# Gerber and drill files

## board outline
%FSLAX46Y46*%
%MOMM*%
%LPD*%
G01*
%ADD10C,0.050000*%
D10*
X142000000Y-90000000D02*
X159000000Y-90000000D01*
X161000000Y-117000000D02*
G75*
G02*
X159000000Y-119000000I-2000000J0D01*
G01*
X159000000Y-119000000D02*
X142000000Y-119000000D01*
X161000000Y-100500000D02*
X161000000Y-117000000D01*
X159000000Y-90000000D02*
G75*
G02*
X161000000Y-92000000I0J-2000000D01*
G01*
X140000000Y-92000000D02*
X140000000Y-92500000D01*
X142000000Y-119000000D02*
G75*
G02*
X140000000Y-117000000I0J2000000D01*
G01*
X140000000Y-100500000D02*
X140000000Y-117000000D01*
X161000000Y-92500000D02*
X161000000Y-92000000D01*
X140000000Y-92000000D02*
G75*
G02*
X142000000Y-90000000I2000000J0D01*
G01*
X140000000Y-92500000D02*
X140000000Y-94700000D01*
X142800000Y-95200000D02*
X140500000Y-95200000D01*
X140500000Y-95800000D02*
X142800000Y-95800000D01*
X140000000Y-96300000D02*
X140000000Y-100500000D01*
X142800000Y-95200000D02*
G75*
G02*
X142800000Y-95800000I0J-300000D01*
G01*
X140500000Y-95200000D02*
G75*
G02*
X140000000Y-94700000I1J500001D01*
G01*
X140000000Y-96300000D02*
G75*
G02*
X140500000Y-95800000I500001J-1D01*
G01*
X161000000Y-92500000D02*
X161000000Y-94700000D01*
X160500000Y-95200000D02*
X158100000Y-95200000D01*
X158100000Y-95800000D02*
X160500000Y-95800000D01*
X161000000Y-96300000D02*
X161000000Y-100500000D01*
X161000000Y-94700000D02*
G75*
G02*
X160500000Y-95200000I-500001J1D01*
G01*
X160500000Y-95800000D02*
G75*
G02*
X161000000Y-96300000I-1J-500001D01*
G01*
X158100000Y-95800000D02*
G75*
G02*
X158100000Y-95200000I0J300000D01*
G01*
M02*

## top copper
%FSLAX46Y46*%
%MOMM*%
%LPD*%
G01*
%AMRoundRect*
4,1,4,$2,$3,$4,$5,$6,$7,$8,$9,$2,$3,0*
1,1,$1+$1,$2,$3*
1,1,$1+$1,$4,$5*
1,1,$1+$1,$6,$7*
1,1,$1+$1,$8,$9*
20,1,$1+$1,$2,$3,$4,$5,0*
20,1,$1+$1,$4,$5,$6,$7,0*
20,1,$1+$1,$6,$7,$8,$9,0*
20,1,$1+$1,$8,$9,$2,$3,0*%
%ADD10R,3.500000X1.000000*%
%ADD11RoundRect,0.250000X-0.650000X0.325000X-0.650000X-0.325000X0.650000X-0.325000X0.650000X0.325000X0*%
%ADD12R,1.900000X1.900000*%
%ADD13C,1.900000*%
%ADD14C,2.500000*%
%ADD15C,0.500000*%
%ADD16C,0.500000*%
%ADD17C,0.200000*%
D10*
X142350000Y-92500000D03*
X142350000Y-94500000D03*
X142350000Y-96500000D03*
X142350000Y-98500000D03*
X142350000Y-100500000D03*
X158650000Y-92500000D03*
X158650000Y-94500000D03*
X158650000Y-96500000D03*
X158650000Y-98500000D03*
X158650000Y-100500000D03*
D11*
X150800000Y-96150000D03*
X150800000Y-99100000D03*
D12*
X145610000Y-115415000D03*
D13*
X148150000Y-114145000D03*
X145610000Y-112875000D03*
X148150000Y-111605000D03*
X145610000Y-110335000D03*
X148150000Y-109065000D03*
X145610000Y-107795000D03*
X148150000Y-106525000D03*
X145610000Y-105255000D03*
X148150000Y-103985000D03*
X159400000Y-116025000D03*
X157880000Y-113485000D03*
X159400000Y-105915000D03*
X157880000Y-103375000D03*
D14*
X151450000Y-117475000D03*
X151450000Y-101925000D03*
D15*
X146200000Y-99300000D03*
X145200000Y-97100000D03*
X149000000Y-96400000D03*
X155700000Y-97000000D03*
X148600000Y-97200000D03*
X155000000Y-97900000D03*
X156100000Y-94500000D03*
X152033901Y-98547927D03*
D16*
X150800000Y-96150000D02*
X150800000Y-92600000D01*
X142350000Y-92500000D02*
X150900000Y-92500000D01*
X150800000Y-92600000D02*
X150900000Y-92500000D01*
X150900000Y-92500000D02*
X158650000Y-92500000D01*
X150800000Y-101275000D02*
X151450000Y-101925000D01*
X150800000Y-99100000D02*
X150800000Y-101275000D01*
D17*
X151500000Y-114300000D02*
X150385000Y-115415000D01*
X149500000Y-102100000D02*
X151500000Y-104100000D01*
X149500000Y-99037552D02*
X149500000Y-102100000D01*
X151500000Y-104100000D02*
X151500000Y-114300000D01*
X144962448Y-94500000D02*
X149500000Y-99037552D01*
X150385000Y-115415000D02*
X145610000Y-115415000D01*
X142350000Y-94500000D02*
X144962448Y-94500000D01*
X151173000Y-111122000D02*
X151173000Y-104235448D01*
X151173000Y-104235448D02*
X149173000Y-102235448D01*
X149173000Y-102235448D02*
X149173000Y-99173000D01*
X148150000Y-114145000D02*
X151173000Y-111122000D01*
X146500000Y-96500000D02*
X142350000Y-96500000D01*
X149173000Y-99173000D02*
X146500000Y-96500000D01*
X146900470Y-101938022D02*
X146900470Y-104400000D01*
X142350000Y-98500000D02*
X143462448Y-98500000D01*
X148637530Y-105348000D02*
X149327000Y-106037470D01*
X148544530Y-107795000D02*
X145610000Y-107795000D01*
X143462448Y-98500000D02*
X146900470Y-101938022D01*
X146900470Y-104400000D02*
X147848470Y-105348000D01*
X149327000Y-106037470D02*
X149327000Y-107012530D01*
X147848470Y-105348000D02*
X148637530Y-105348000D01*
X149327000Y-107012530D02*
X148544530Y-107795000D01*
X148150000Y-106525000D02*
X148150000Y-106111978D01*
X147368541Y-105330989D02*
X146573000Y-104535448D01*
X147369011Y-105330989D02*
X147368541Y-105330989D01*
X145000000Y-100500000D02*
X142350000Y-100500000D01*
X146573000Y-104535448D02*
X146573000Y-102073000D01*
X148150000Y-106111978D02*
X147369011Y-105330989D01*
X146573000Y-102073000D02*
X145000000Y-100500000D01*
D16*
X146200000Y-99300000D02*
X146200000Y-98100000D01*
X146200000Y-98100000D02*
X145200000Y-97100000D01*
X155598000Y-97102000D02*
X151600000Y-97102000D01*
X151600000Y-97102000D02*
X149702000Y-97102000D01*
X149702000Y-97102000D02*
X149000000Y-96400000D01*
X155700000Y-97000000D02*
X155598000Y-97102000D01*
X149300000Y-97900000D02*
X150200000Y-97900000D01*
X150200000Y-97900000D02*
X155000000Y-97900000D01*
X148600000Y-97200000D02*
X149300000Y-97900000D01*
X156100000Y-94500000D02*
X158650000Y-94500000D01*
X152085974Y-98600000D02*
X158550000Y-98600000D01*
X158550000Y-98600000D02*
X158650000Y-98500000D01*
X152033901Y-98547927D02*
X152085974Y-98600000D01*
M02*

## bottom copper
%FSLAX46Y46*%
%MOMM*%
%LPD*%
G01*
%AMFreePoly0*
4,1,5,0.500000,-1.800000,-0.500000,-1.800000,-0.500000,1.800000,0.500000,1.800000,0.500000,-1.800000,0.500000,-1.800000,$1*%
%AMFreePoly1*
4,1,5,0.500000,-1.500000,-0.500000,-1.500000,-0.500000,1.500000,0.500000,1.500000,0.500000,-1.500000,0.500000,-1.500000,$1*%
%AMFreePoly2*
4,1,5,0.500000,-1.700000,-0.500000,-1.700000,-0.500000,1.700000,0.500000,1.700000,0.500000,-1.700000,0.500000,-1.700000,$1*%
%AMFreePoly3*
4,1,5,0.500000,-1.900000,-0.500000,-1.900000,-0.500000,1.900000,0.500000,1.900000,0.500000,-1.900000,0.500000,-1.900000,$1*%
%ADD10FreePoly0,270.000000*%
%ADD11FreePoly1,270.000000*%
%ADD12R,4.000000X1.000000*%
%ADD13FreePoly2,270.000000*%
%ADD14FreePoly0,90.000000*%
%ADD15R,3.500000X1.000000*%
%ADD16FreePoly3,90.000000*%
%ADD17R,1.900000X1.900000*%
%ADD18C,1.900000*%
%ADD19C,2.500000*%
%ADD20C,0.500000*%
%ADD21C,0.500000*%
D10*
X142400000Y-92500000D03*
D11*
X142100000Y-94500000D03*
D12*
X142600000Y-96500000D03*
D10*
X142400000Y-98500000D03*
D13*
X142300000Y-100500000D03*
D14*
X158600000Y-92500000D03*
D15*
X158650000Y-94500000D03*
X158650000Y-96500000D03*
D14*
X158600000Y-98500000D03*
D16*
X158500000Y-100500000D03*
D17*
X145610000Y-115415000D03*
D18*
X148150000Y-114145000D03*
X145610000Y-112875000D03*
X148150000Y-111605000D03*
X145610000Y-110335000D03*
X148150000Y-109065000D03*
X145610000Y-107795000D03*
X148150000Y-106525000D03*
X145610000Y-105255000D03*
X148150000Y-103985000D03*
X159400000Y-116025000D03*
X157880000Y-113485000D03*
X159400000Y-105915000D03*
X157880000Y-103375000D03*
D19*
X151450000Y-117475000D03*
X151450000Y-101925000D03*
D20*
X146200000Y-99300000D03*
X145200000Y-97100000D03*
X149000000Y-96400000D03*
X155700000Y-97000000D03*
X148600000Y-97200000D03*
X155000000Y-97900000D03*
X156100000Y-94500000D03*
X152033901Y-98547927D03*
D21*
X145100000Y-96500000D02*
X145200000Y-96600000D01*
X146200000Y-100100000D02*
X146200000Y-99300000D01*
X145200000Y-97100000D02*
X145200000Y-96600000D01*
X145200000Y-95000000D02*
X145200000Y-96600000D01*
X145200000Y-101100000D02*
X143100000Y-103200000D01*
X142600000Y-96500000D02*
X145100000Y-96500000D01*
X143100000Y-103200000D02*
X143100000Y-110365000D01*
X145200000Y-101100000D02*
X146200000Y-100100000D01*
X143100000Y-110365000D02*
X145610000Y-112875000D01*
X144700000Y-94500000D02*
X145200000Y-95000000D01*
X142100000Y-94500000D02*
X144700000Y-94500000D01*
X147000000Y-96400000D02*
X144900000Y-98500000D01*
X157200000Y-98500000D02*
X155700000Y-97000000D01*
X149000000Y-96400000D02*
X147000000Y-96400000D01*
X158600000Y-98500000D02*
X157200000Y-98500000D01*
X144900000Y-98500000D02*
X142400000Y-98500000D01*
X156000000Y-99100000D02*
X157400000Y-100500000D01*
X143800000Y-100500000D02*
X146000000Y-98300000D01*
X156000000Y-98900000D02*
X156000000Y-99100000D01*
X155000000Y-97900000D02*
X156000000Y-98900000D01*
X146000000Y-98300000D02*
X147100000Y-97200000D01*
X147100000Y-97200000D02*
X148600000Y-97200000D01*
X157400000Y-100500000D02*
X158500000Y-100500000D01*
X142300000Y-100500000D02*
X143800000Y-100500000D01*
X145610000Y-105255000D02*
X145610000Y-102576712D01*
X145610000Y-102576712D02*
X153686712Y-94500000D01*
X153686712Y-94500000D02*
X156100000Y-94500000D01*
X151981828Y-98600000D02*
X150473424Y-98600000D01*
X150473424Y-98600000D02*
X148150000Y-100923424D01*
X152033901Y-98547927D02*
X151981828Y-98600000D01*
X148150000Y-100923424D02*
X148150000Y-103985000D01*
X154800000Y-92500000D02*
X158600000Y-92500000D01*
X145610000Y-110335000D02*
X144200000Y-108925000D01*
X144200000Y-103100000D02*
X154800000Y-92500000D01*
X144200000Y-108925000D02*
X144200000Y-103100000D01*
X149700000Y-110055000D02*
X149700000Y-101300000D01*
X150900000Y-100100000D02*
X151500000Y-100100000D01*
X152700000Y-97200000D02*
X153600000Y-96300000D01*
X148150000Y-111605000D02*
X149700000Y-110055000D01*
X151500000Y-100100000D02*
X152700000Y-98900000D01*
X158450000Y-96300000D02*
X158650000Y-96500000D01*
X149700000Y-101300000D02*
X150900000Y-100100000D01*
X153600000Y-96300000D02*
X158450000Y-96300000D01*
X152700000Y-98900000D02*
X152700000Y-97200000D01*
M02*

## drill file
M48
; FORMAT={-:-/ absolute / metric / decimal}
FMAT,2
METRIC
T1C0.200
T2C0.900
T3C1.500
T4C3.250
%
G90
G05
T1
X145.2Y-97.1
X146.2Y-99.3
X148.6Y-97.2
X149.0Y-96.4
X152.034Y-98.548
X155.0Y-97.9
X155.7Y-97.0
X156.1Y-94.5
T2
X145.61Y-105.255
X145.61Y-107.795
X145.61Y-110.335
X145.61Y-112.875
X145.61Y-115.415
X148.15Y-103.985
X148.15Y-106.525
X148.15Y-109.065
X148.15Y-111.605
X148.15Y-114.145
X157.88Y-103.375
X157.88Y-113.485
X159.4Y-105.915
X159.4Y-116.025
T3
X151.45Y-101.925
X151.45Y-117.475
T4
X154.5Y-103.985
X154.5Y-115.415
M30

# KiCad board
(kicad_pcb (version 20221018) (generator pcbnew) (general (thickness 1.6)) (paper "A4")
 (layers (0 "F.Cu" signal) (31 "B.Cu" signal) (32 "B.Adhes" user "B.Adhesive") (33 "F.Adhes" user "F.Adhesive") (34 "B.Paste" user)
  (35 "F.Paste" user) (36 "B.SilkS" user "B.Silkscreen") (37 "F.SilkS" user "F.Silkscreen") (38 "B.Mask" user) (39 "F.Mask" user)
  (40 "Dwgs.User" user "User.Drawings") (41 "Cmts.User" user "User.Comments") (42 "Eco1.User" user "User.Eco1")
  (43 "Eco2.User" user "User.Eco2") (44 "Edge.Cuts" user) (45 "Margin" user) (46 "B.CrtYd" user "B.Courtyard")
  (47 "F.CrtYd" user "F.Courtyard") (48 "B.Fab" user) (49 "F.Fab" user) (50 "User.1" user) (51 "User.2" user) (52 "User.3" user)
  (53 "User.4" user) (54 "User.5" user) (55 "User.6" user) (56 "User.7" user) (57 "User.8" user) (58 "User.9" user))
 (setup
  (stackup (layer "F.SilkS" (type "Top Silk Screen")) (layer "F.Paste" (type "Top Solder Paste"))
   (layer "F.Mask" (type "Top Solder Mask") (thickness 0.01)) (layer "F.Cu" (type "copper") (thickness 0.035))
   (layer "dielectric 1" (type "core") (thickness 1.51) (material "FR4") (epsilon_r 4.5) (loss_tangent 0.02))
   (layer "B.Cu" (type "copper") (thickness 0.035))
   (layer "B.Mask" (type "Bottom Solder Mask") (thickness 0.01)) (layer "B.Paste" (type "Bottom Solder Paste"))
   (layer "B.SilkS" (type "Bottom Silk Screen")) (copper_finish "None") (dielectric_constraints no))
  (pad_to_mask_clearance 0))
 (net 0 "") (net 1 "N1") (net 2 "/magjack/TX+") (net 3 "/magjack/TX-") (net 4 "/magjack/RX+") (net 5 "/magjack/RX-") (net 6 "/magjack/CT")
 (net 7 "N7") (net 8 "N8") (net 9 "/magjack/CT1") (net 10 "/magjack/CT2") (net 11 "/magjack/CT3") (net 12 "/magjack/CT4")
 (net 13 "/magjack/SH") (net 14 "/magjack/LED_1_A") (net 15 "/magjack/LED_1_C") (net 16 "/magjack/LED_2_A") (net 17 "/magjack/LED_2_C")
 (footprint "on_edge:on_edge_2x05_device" (layer "F.Cu") (at 140 96.5 -90)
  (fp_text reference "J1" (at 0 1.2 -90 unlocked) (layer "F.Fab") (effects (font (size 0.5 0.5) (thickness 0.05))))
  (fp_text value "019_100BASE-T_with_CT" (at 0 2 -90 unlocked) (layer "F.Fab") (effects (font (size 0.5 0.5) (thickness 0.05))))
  (fp_line (start -4 0) (end -1.8 0) (stroke (width 0.05) (type solid)) (layer "Edge.Cuts"))
  (fp_line (start -1.3 -2.8) (end -1.3 -0.5) (stroke (width 0.05) (type solid)) (layer "Edge.Cuts"))
  (fp_line (start -0.7 -0.5) (end -0.7 -2.8) (stroke (width 0.05) (type solid)) (layer "Edge.Cuts"))
  (fp_line (start -0.2 0) (end 4 0) (stroke (width 0.05) (type solid)) (layer "Edge.Cuts"))
  (fp_arc (start -1.3 -2.8) (mid -1 -3.1) (end -0.7 -2.8) (stroke (width 0.05) (type solid)) (layer "Edge.Cuts"))
  (fp_arc (start -1.3 -0.5) (mid -1.446447 -0.146447) (end -1.8 0) (stroke (width 0.05) (type solid)) (layer "Edge.Cuts"))
  (fp_arc (start -0.2 0) (mid -0.553553 -0.146447) (end -0.7 -0.5) (stroke (width 0.05) (type solid)) (layer "Edge.Cuts"))
  (pad "1" smd rect (at -4 -2.35 90) (size 1 3.5) (layers "F.Cu" "F.Mask") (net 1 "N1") (zone_connect 0))
  (pad "2" smd rect (at -2 -2.35 270) (size 1 3.5) (layers "F.Cu" "F.Mask") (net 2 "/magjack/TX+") (zone_connect 0))
  (pad "3" smd rect (at 0 -2.35 270) (size 1 3.5) (layers "F.Cu" "F.Mask") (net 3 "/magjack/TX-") (zone_connect 0))
  (pad "4" smd rect (at 2 -2.35 90) (size 1 3.5) (layers "F.Cu" "F.Mask") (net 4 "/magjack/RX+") (zone_connect 0))
  (pad "5" smd rect (at 4 -2.35 90) (size 1 3.5) (layers "F.Cu" "F.Mask") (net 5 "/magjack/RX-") (zone_connect 0))
  (pad "6" smd custom (at -4 -2.4 270) (size 1 3.6) (layers "B.Cu" "B.Mask") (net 1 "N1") (zone_connect 0)
   (options (clearance outline) (anchor rect)) (primitives))
  (pad "7" smd custom (at -2 -2.1 270) (size 1 3) (layers "B.Cu" "B.Mask") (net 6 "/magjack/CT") (zone_connect 0)
   (options (clearance outline) (anchor rect)) (primitives))
  (pad "8" smd rect (at 0 -2.6 270) (size 1 4) (layers "B.Cu" "B.Mask") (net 6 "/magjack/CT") (zone_connect 0))
  (pad "9" smd custom (at 2 -2.4 270) (size 1 3.6) (layers "B.Cu" "B.Mask") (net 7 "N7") (zone_connect 0)
   (options (clearance outline) (anchor rect)) (primitives))
  (pad "10" smd custom (at 4 -2.3 270) (size 1 3.4) (layers "B.Cu" "B.Mask") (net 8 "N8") (zone_connect 0)
   (options (clearance outline) (anchor rect)) (primitives))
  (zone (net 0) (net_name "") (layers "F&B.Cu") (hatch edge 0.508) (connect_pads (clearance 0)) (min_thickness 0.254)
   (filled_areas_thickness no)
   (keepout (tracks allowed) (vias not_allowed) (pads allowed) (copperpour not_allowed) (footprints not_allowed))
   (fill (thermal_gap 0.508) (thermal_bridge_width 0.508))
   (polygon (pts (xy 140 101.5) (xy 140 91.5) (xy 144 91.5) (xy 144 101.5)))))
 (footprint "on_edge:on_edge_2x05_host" (layer "F.Cu") (at 161 96.5 -90)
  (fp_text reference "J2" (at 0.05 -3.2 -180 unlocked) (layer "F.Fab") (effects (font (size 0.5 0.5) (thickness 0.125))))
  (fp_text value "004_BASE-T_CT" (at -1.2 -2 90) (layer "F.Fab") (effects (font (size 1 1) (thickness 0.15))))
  (fp_line (start -4 0) (end -1.8 0) (stroke (width 0.05) (type solid)) (layer "Edge.Cuts"))
  (fp_line (start -1.3 0.5) (end -1.3 2.9) (stroke (width 0.05) (type solid)) (layer "Edge.Cuts"))
  (fp_line (start -0.7 2.9) (end -0.7 0.5) (stroke (width 0.05) (type solid)) (layer "Edge.Cuts"))
  (fp_line (start -0.2 0) (end 4 0) (stroke (width 0.05) (type solid)) (layer "Edge.Cuts"))
  (fp_arc (start -1.8 0) (mid -1.446447 0.146447) (end -1.3 0.5) (stroke (width 0.05) (type solid)) (layer "Edge.Cuts"))
  (fp_arc (start -0.7 0.5) (mid -0.553553 0.146447) (end -0.2 0) (stroke (width 0.05) (type solid)) (layer "Edge.Cuts"))
  (fp_arc (start -0.7 2.9) (mid -1 3.2) (end -1.3 2.9) (stroke (width 0.05) (type solid)) (layer "Edge.Cuts"))
  (pad "1" smd rect (at -4 2.35 270) (size 1 3.5) (layers "F.Cu" "F.Mask") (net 1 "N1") (zone_connect 0))
  (pad "2" smd rect (at -2 2.35 270) (size 1 3.5) (layers "F.Cu" "F.Mask") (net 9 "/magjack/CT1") (zone_connect 0))
  (pad "3" smd rect (at 0 2.35 270) (size 1 3.5) (layers "F.Cu" "F.Mask") (zone_connect 0))
  (pad "4" smd rect (at 2 2.35 270) (size 1 3.5) (layers "F.Cu" "F.Mask") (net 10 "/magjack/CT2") (zone_connect 0))
  (pad "5" smd rect (at 4 2.35 270) (size 1 3.5) (layers "F.Cu" "F.Mask") (zone_connect 0))
  (pad "6" smd custom (at -4 2.4 90) (size 1 3.6) (layers "B.Cu" "B.Mask") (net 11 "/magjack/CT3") (zone_connect 0)
   (options (clearance outline) (anchor rect)) (primitives))
  (pad "7" smd rect (at -2 2.35 90) (size 1 3.5) (layers "B.Cu" "B.Mask") (zone_connect 0))
  (pad "8" smd rect (at 0 2.35 90) (size 1 3.5) (layers "B.Cu" "B.Mask") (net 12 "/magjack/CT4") (zone_connect 0))
  (pad "9" smd custom (at 2 2.4 90) (size 1 3.6) (layers "B.Cu" "B.Mask") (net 7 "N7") (zone_connect 0)
   (options (clearance outline) (anchor rect)) (primitives))
  (pad "10" smd custom (at 4 2.5 90) (size 1 3.8) (layers "B.Cu" "B.Mask") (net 8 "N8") (zone_connect 0)
   (options (clearance outline) (anchor rect)) (primitives))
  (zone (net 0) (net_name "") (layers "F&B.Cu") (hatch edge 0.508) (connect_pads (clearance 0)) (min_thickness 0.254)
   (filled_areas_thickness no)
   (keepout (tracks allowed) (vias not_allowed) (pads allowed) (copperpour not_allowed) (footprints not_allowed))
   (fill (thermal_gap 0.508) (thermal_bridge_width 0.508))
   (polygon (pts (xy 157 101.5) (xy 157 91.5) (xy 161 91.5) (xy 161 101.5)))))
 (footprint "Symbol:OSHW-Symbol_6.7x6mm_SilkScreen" (layer "F.Cu") (at 150.8 93.1)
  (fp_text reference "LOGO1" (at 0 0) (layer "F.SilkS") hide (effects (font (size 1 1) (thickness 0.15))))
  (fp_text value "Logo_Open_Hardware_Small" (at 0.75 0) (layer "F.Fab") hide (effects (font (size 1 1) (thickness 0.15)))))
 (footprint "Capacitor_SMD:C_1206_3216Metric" (layer "F.Cu") (at 150.8 97.625 -90)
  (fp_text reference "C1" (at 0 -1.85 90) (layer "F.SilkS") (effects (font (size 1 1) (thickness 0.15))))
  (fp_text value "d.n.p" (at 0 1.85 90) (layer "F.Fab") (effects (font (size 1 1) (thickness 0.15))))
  (pad "1" smd roundrect (at -1.475 0 270) (size 1.15 1.8) (layers "F.Cu" "F.Paste" "F.Mask") (roundrect_rratio 0.217391) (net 1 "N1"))
  (pad "2" smd roundrect (at 1.475 0 270) (size 1.15 1.8) (layers "F.Cu" "F.Paste" "F.Mask") (roundrect_rratio 0.217391)
   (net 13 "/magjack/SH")))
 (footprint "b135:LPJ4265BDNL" (layer "F.Cu") (at 145.61 115.415 90)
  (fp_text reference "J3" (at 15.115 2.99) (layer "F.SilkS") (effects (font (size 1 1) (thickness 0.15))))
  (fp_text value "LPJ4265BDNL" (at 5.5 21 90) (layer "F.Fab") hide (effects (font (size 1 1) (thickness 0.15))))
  (pad "" np_thru_hole circle (at 0 8.89 90) (size 3.25 3.25) (drill 3.25) (layers "*.Cu" "*.Mask"))
  (pad "" np_thru_hole circle (at 11.43 8.89 90) (size 3.25 3.25) (drill 3.25) (layers "*.Cu" "*.Mask"))
  (pad "1" thru_hole rect (at 0 0 90) (size 1.9 1.9) (drill 0.9) (layers "*.Cu" "*.Mask") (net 2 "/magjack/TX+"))
  (pad "2" thru_hole circle (at 1.27 2.54 90) (size 1.9 1.9) (drill 0.9) (layers "*.Cu" "*.Mask") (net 3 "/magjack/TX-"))
  (pad "3" thru_hole circle (at 2.54 0 90) (size 1.9 1.9) (drill 0.9) (layers "*.Cu" "*.Mask") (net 6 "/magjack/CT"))
  (pad "4" thru_hole circle (at 3.81 2.54 90) (size 1.9 1.9) (drill 0.9) (layers "*.Cu" "*.Mask") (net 12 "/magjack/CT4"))
  (pad "5" thru_hole circle (at 5.08 0 90) (size 1.9 1.9) (drill 0.9) (layers "*.Cu" "*.Mask") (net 11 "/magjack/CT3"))
  (pad "6" thru_hole circle (at 6.35 2.54 90) (size 1.9 1.9) (drill 0.9) (layers "*.Cu" "*.Mask"))
  (pad "7" thru_hole circle (at 7.62 0 90) (size 1.9 1.9) (drill 0.9) (layers "*.Cu" "*.Mask") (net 4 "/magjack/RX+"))
  (pad "8" thru_hole circle (at 8.89 2.54 90) (size 1.9 1.9) (drill 0.9) (layers "*.Cu" "*.Mask") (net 5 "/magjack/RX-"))
  (pad "9" thru_hole circle (at 10.16 0 90) (size 1.9 1.9) (drill 0.9) (layers "*.Cu" "*.Mask") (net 9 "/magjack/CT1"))
  (pad "10" thru_hole circle (at 11.43 2.54 90) (size 1.9 1.9) (drill 0.9) (layers "*.Cu" "*.Mask") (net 10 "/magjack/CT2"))
  (pad "11" thru_hole circle (at -0.61 13.79 90) (size 1.9 1.9) (drill 0.9) (layers "*.Cu" "*.Mask") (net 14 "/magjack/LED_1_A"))
  (pad "12" thru_hole circle (at 1.93 12.27 90) (size 1.9 1.9) (drill 0.9) (layers "*.Cu" "*.Mask") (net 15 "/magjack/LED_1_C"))
  (pad "13" thru_hole circle (at 9.5 13.79 90) (size 1.9 1.9) (drill 0.9) (layers "*.Cu" "*.Mask") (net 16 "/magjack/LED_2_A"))
  (pad "14" thru_hole circle (at 12.04 12.27 90) (size 1.9 1.9) (drill 0.9) (layers "*.Cu" "*.Mask") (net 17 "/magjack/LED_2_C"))
  (pad "SH" thru_hole circle (at -2.06 5.84 90) (size 2.5 2.5) (drill 1.5) (layers "*.Cu" "*.Mask") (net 13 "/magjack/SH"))
  (pad "SH" thru_hole circle (at 13.49 5.84 90) (size 2.5 2.5) (drill 1.5) (layers "*.Cu" "*.Mask") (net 13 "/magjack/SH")))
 (gr_line (start 142 90) (end 159 90) (stroke (width 0.05) (type solid)) (layer "Edge.Cuts"))
 (gr_arc (start 161 117) (mid 160.414214 118.414214) (end 159 119) (stroke (width 0.05) (type solid)) (layer "Edge.Cuts"))
 (gr_line (start 159 119) (end 142 119) (stroke (width 0.05) (type solid)) (layer "Edge.Cuts"))
 (gr_line (start 161 100.5) (end 161 117) (stroke (width 0.05) (type solid)) (layer "Edge.Cuts"))
 (gr_arc (start 159 90) (mid 160.414214 90.585786) (end 161 92) (stroke (width 0.05) (type solid)) (layer "Edge.Cuts"))
 (gr_line (start 140 92) (end 140 92.5) (stroke (width 0.05) (type solid)) (layer "Edge.Cuts"))
 (gr_arc (start 142 119) (mid 140.585786 118.414214) (end 140 117) (stroke (width 0.05) (type solid)) (layer "Edge.Cuts"))
 (gr_line (start 140 100.5) (end 140 117) (stroke (width 0.05) (type solid)) (layer "Edge.Cuts"))
 (gr_line (start 161 92.5) (end 161 92) (stroke (width 0.05) (type solid)) (layer "Edge.Cuts"))
 (gr_arc (start 140 92) (mid 140.585786 90.585786) (end 142 90) (stroke (width 0.05) (type solid)) (layer "Edge.Cuts"))
 (segment (start 150.8 96.15) (end 150.8 92.6) (width 0.5) (layer "F.Cu") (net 1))
 (segment (start 142.35 92.5) (end 150.9 92.5) (width 0.5) (layer "F.Cu") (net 1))
 (segment (start 150.8 92.6) (end 150.9 92.5) (width 0.5) (layer "F.Cu") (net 1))
 (segment (start 150.9 92.5) (end 158.65 92.5) (width 0.5) (layer "F.Cu") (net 1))
 (segment (start 150.8 101.275) (end 151.45 101.925) (width 0.5) (layer "F.Cu") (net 13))
 (segment (start 150.8 99.1) (end 150.8 101.275) (width 0.5) (layer "F.Cu") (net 13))
 (segment (start 151.5 114.3) (end 150.385 115.415) (width 0.2) (layer "F.Cu") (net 2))
 (segment (start 149.5 102.1) (end 151.5 104.1) (width 0.2) (layer "F.Cu") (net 2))
 (segment (start 149.5 99.037552) (end 149.5 102.1) (width 0.2) (layer "F.Cu") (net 2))
 (segment (start 151.5 104.1) (end 151.5 114.3) (width 0.2) (layer "F.Cu") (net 2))
 (segment (start 144.962448 94.5) (end 149.5 99.037552) (width 0.2) (layer "F.Cu") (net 2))
 (segment (start 150.385 115.415) (end 145.61 115.415) (width 0.2) (layer "F.Cu") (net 2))
 (segment (start 142.35 94.5) (end 144.962448 94.5) (width 0.2) (layer "F.Cu") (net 2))
 (segment (start 151.173 111.122) (end 151.173 104.235448) (width 0.2) (layer "F.Cu") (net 3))
 (segment (start 151.173 104.235448) (end 149.173 102.235448) (width 0.2) (layer "F.Cu") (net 3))
 (segment (start 149.173 102.235448) (end 149.173 99.173) (width 0.2) (layer "F.Cu") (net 3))
 (segment (start 148.15 114.145) (end 151.173 111.122) (width 0.2) (layer "F.Cu") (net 3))
 (segment (start 146.5 96.5) (end 142.35 96.5) (width 0.2) (layer "F.Cu") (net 3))
 (segment (start 149.173 99.173) (end 146.5 96.5) (width 0.2) (layer "F.Cu") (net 3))
 (segment (start 146.90047 101.938022) (end 146.90047 104.4) (width 0.2) (layer "F.Cu") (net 4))
 (segment (start 142.35 98.5) (end 143.462448 98.5) (width 0.2) (layer "F.Cu") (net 4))
 (segment (start 148.63753 105.348) (end 149.327 106.03747) (width 0.2) (layer "F.Cu") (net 4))
 (segment (start 148.54453 107.795) (end 145.61 107.795) (width 0.2) (layer "F.Cu") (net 4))
 (segment (start 143.462448 98.5) (end 146.90047 101.938022) (width 0.2) (layer "F.Cu") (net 4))
 (segment (start 146.90047 104.4) (end 147.84847 105.348) (width 0.2) (layer "F.Cu") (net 4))
 (segment (start 149.327 106.03747) (end 149.327 107.01253) (width 0.2) (layer "F.Cu") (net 4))
 (segment (start 147.84847 105.348) (end 148.63753 105.348) (width 0.2) (layer "F.Cu") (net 4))
 (segment (start 149.327 107.01253) (end 148.54453 107.795) (width 0.2) (layer "F.Cu") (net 4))
 (segment (start 148.15 106.525) (end 148.15 106.111978) (width 0.2) (layer "F.Cu") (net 5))
 (segment (start 147.368541 105.330989) (end 146.573 104.535448) (width 0.2) (layer "F.Cu") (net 5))
 (segment (start 147.369011 105.330989) (end 147.368541 105.330989) (width 0.2) (layer "F.Cu") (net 5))
 (segment (start 145 100.5) (end 142.35 100.5) (width 0.2) (layer "F.Cu") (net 5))
 (segment (start 146.573 104.535448) (end 146.573 102.073) (width 0.2) (layer "F.Cu") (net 5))
 (segment (start 148.15 106.111978) (end 147.369011 105.330989) (width 0.2) (layer "F.Cu") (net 5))
 (segment (start 146.573 102.073) (end 145 100.5) (width 0.2) (layer "F.Cu") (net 5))
 (segment (start 146.2 99.3) (end 146.2 98.1) (width 0.5) (layer "F.Cu") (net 6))
 (segment (start 146.2 98.1) (end 145.2 97.1) (width 0.5) (layer "F.Cu") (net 6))
 (via (at 146.2 99.3) (size 0.5) (drill 0.2) (layers "F.Cu" "B.Cu") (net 6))
 (via (at 145.2 97.1) (size 0.5) (drill 0.2) (layers "F.Cu" "B.Cu") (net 6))
 (segment (start 145.1 96.5) (end 145.2 96.6) (width 0.5) (layer "B.Cu") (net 6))
 (segment (start 146.2 100.1) (end 146.2 99.3) (width 0.5) (layer "B.Cu") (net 6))
 (segment (start 145.2 97.1) (end 145.2 96.6) (width 0.5) (layer "B.Cu") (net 6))
 (segment (start 145.2 95) (end 145.2 96.6) (width 0.5) (layer "B.Cu") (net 6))
 (segment (start 145.2 101.1) (end 143.1 103.2) (width 0.5) (layer "B.Cu") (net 6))
 (segment (start 142.6 96.5) (end 145.1 96.5) (width 0.5) (layer "B.Cu") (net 6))
 (segment (start 143.1 103.2) (end 143.1 110.365) (width 0.5) (layer "B.Cu") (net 6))
 (segment (start 145.2 101.1) (end 146.2 100.1) (width 0.5) (layer "B.Cu") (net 6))
 (segment (start 143.1 110.365) (end 145.61 112.875) (width 0.5) (layer "B.Cu") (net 6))
 (segment (start 144.7 94.5) (end 145.2 95) (width 0.5) (layer "B.Cu") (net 6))
 (segment (start 142.1 94.5) (end 144.7 94.5) (width 0.5) (layer "B.Cu") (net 6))
 (segment (start 155.598 97.102) (end 151.6 97.102) (width 0.5) (layer "F.Cu") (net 7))
 (segment (start 151.6 97.102) (end 149.702 97.102) (width 0.5) (layer "F.Cu") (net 7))
 (segment (start 149.702 97.102) (end 149 96.4) (width 0.5) (layer "F.Cu") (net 7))
 (segment (start 155.7 97) (end 155.598 97.102) (width 0.5) (layer "F.Cu") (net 7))
 (via (at 149 96.4) (size 0.5) (drill 0.2) (layers "F.Cu" "B.Cu") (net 7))
 (via (at 155.7 97) (size 0.5) (drill 0.2) (layers "F.Cu" "B.Cu") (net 7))
 (segment (start 147 96.4) (end 144.9 98.5) (width 0.5) (layer "B.Cu") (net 7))
 (segment (start 157.2 98.5) (end 155.7 97) (width 0.5) (layer "B.Cu") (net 7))
 (segment (start 149 96.4) (end 147 96.4) (width 0.5) (layer "B.Cu") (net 7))
 (segment (start 158.6 98.5) (end 157.2 98.5) (width 0.5) (layer "B.Cu") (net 7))
 (segment (start 144.9 98.5) (end 142.4 98.5) (width 0.5) (layer "B.Cu") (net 7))
 (segment (start 149.3 97.9) (end 150.2 97.9) (width 0.5) (layer "F.Cu") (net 8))
 (segment (start 150.2 97.9) (end 155 97.9) (width 0.5) (layer "F.Cu") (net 8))
 (segment (start 148.6 97.2) (end 149.3 97.9) (width 0.5) (layer "F.Cu") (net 8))
 (via (at 148.6 97.2) (size 0.5) (drill 0.2) (layers "F.Cu" "B.Cu") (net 8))
 (via (at 155 97.9) (size 0.5) (drill 0.2) (layers "F.Cu" "B.Cu") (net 8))
 (segment (start 156 99.1) (end 157.4 100.5) (width 0.5) (layer "B.Cu") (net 8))
 (segment (start 143.8 100.5) (end 146 98.3) (width 0.5) (layer "B.Cu") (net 8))
 (segment (start 156 98.9) (end 156 99.1) (width 0.5) (layer "B.Cu") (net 8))
 (segment (start 155 97.9) (end 156 98.9) (width 0.5) (layer "B.Cu") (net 8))
 (segment (start 146 98.3) (end 147.1 97.2) (width 0.5) (layer "B.Cu") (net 8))
 (segment (start 147.1 97.2) (end 148.6 97.2) (width 0.5) (layer "B.Cu") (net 8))
 (segment (start 157.4 100.5) (end 158.5 100.5) (width 0.5) (layer "B.Cu") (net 8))
 (segment (start 142.3 100.5) (end 143.8 100.5) (width 0.5) (layer "B.Cu") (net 8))
 (segment (start 156.1 94.5) (end 158.65 94.5) (width 0.5) (layer "F.Cu") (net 9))
 (via (at 156.1 94.5) (size 0.5) (drill 0.2) (layers "F.Cu" "B.Cu") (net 9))
 (segment (start 145.61 105.255) (end 145.61 102.576712) (width 0.5) (layer "B.Cu") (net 9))
 (segment (start 145.61 102.576712) (end 153.686712 94.5) (width 0.5) (layer "B.Cu") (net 9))
 (segment (start 153.686712 94.5) (end 156.1 94.5) (width 0.5) (layer "B.Cu") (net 9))
 (segment (start 152.085974 98.6) (end 158.55 98.6) (width 0.5) (layer "F.Cu") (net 10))
 (segment (start 158.55 98.6) (end 158.65 98.5) (width 0.5) (layer "F.Cu") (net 10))
 (segment (start 152.033901 98.547927) (end 152.085974 98.6) (width 0.5) (layer "F.Cu") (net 10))
 (via (at 152.033901 98.547927) (size 0.5) (drill 0.2) (layers "F.Cu" "B.Cu") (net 10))
 (segment (start 151.981828 98.6) (end 150.473424 98.6) (width 0.5) (layer "B.Cu") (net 10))
 (segment (start 150.473424 98.6) (end 148.15 100.923424) (width 0.5) (layer "B.Cu") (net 10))
 (segment (start 152.033901 98.547927) (end 151.981828 98.6) (width 0.5) (layer "B.Cu") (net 10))
 (segment (start 148.15 100.923424) (end 148.15 103.985) (width 0.5) (layer "B.Cu") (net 10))
 (segment (start 154.8 92.5) (end 158.6 92.5) (width 0.5) (layer "B.Cu") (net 11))
 (segment (start 145.61 110.335) (end 144.2 108.925) (width 0.5) (layer "B.Cu") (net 11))
 (segment (start 144.2 103.1) (end 154.8 92.5) (width 0.5) (layer "B.Cu") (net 11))
 (segment (start 144.2 108.925) (end 144.2 103.1) (width 0.5) (layer "B.Cu") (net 11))
 (segment (start 149.7 110.055) (end 149.7 101.3) (width 0.5) (layer "B.Cu") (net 12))
 (segment (start 150.9 100.1) (end 151.5 100.1) (width 0.5) (layer "B.Cu") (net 12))
 (segment (start 152.7 97.2) (end 153.6 96.3) (width 0.5) (layer "B.Cu") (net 12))
 (segment (start 148.15 111.605) (end 149.7 110.055) (width 0.5) (layer "B.Cu") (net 12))
 (segment (start 151.5 100.1) (end 152.7 98.9) (width 0.5) (layer "B.Cu") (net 12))
 (segment (start 158.45 96.3) (end 158.65 96.5) (width 0.5) (layer "B.Cu") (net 12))
 (segment (start 149.7 101.3) (end 150.9 100.1) (width 0.5) (layer "B.Cu") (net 12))
 (segment (start 153.6 96.3) (end 158.45 96.3) (width 0.5) (layer "B.Cu") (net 12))
 (segment (start 152.7 98.9) (end 152.7 97.2) (width 0.5) (layer "B.Cu") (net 12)))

